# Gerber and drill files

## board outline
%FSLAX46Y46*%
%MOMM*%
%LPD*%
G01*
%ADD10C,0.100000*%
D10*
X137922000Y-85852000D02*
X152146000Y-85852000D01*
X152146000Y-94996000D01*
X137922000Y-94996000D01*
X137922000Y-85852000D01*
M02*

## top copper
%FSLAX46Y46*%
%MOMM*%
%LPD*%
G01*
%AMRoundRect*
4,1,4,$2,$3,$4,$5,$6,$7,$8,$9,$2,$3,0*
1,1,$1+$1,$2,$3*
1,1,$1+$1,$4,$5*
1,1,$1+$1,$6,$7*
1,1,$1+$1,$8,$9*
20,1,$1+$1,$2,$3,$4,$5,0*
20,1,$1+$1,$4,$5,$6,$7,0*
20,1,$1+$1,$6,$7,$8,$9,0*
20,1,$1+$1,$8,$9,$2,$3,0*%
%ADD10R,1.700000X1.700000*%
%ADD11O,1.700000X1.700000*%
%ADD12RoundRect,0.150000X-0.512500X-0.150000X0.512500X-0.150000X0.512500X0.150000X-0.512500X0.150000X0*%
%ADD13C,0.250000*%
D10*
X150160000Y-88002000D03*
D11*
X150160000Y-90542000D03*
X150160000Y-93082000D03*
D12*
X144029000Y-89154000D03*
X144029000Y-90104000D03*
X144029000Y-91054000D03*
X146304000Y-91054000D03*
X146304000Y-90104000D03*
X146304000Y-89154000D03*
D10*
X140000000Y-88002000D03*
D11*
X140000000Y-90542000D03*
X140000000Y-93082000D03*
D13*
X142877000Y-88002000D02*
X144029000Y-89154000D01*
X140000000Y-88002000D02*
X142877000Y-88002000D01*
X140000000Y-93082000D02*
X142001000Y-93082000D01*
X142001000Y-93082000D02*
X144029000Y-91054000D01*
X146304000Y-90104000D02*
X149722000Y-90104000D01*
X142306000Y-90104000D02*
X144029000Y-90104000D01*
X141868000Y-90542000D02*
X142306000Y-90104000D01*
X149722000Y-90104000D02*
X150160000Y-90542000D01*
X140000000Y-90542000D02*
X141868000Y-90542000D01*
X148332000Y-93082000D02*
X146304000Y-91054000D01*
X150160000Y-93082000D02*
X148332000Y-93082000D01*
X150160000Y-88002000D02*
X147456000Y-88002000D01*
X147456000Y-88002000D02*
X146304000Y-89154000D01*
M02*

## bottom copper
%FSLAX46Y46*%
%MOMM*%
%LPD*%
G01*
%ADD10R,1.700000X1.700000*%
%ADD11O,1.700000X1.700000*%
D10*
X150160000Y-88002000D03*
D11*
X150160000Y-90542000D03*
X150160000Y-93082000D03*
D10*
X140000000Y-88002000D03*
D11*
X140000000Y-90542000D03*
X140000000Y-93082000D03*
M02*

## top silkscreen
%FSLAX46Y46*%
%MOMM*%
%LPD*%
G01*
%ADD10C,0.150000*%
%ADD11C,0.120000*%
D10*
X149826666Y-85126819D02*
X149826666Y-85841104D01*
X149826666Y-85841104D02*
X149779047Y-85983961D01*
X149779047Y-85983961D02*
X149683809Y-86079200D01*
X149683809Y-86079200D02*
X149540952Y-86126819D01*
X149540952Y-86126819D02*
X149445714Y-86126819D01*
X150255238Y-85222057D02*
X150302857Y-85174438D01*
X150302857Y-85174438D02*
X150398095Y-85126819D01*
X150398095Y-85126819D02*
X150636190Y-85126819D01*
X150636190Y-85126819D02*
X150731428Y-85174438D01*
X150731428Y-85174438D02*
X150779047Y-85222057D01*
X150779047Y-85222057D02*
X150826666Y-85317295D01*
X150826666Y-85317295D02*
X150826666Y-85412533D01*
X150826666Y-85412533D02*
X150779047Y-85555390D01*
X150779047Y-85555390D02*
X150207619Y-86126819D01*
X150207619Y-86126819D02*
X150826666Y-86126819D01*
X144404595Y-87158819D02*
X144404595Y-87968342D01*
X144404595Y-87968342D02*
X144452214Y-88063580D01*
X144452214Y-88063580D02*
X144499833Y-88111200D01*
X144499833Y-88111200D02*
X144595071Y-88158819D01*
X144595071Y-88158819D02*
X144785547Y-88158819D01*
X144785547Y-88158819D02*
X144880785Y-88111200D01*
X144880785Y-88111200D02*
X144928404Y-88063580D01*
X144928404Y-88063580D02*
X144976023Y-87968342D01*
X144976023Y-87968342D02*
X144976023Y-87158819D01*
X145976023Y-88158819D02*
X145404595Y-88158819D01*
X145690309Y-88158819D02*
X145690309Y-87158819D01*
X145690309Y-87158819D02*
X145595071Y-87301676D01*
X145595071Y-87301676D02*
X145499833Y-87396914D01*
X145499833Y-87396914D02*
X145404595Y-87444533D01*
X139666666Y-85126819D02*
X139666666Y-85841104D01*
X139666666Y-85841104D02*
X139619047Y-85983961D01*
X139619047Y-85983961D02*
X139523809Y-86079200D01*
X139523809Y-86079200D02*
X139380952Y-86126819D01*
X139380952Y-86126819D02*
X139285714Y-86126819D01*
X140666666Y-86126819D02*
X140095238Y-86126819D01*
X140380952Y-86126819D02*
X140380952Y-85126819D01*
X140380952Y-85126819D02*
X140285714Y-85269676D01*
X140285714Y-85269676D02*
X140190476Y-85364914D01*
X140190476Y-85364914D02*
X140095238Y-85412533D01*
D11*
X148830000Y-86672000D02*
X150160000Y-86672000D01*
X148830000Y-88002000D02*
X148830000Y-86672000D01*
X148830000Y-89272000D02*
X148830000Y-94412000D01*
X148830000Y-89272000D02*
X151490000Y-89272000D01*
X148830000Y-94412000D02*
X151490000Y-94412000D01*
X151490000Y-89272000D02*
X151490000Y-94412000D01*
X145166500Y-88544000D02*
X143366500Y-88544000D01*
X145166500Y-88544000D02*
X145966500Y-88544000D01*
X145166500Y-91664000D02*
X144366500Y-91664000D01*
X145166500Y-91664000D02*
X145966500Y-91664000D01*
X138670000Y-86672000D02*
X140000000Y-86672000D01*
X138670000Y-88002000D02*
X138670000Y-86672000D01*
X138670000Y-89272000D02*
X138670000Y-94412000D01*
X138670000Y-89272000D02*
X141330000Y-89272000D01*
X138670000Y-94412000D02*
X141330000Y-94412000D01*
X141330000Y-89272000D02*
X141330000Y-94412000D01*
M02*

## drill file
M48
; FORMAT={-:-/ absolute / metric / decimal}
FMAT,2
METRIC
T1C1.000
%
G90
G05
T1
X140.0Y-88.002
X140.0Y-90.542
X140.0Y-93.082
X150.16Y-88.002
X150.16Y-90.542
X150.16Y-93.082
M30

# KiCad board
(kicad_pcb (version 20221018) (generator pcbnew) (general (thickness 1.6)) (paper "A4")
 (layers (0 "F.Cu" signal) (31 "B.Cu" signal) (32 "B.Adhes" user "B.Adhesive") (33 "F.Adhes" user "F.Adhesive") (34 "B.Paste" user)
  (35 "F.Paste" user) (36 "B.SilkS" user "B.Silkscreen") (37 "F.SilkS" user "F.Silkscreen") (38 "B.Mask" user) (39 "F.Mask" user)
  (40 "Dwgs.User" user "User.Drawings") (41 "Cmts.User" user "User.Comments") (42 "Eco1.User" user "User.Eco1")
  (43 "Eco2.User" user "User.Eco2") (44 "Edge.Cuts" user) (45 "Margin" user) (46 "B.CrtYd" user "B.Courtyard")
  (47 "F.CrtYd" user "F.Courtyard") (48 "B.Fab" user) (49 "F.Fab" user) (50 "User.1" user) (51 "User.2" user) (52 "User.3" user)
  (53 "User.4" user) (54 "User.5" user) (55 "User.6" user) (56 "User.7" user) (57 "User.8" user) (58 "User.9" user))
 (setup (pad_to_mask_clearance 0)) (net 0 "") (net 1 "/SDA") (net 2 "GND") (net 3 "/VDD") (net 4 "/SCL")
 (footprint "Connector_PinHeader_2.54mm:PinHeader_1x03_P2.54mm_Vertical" (layer "F.Cu") (at 150.16 88.002)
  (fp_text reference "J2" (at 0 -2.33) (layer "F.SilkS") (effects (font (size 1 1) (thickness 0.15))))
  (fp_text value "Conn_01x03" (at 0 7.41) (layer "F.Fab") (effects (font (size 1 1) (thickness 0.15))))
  (fp_line (start -1.33 -1.33) (end 0 -1.33) (stroke (width 0.12) (type solid)) (layer "F.SilkS"))
  (fp_line (start -1.33 0) (end -1.33 -1.33) (stroke (width 0.12) (type solid)) (layer "F.SilkS"))
  (fp_line (start -1.33 1.27) (end -1.33 6.41) (stroke (width 0.12) (type solid)) (layer "F.SilkS"))
  (fp_line (start -1.33 1.27) (end 1.33 1.27) (stroke (width 0.12) (type solid)) (layer "F.SilkS"))
  (fp_line (start -1.33 6.41) (end 1.33 6.41) (stroke (width 0.12) (type solid)) (layer "F.SilkS"))
  (fp_line (start 1.33 1.27) (end 1.33 6.41) (stroke (width 0.12) (type solid)) (layer "F.SilkS"))
  (pad "1" thru_hole rect (at 0 0) (size 1.7 1.7) (drill 1) (layers "*.Cu" "*.Mask") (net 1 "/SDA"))
  (pad "2" thru_hole oval (at 0 2.54) (size 1.7 1.7) (drill 1) (layers "*.Cu" "*.Mask") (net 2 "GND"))
  (pad "3" thru_hole oval (at 0 5.08) (size 1.7 1.7) (drill 1) (layers "*.Cu" "*.Mask") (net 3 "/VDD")))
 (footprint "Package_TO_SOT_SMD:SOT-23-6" (layer "F.Cu") (at 145.1665 90.104)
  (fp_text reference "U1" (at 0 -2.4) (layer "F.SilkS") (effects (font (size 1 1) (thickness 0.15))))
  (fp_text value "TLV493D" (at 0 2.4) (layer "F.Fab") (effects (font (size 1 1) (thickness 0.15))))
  (fp_line (start 0 -1.56) (end -1.8 -1.56) (stroke (width 0.12) (type solid)) (layer "F.SilkS"))
  (fp_line (start 0 -1.56) (end 0.8 -1.56) (stroke (width 0.12) (type solid)) (layer "F.SilkS"))
  (fp_line (start 0 1.56) (end -0.8 1.56) (stroke (width 0.12) (type solid)) (layer "F.SilkS"))
  (fp_line (start 0 1.56) (end 0.8 1.56) (stroke (width 0.12) (type solid)) (layer "F.SilkS"))
  (pad "1" smd roundrect (at -1.1375 -0.95) (size 1.325 0.6) (layers "F.Cu" "F.Paste" "F.Mask") (roundrect_rratio 0.25) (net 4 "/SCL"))
  (pad "2" smd roundrect (at -1.1375 0) (size 1.325 0.6) (layers "F.Cu" "F.Paste" "F.Mask") (roundrect_rratio 0.25) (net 2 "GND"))
  (pad "3" smd roundrect (at -1.1375 0.95) (size 1.325 0.6) (layers "F.Cu" "F.Paste" "F.Mask") (roundrect_rratio 0.25) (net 2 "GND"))
  (pad "4" smd roundrect (at 1.1375 0.95) (size 1.325 0.6) (layers "F.Cu" "F.Paste" "F.Mask") (roundrect_rratio 0.25) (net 3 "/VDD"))
  (pad "5" smd roundrect (at 1.1375 0) (size 1.325 0.6) (layers "F.Cu" "F.Paste" "F.Mask") (roundrect_rratio 0.25) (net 2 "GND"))
  (pad "6" smd roundrect (at 1.1375 -0.95) (size 1.325 0.6) (layers "F.Cu" "F.Paste" "F.Mask") (roundrect_rratio 0.25) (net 1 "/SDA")))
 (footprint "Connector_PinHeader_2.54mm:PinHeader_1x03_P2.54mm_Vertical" (layer "F.Cu") (at 140 88.002)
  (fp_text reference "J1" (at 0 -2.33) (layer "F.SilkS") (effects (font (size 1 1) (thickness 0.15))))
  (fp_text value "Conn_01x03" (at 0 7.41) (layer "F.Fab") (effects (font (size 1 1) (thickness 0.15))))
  (fp_line (start -1.33 -1.33) (end 0 -1.33) (stroke (width 0.12) (type solid)) (layer "F.SilkS"))
  (fp_line (start -1.33 0) (end -1.33 -1.33) (stroke (width 0.12) (type solid)) (layer "F.SilkS"))
  (fp_line (start -1.33 1.27) (end -1.33 6.41) (stroke (width 0.12) (type solid)) (layer "F.SilkS"))
  (fp_line (start -1.33 1.27) (end 1.33 1.27) (stroke (width 0.12) (type solid)) (layer "F.SilkS"))
  (fp_line (start -1.33 6.41) (end 1.33 6.41) (stroke (width 0.12) (type solid)) (layer "F.SilkS"))
  (fp_line (start 1.33 1.27) (end 1.33 6.41) (stroke (width 0.12) (type solid)) (layer "F.SilkS"))
  (pad "1" thru_hole rect (at 0 0) (size 1.7 1.7) (drill 1) (layers "*.Cu" "*.Mask") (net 4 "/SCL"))
  (pad "2" thru_hole oval (at 0 2.54) (size 1.7 1.7) (drill 1) (layers "*.Cu" "*.Mask") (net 2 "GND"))
  (pad "3" thru_hole oval (at 0 5.08) (size 1.7 1.7) (drill 1) (layers "*.Cu" "*.Mask") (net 2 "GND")))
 (gr_rect (start 137.922 85.852) (end 152.146 94.996) (stroke (width 0.1) (type default)) (fill none) (layer "Edge.Cuts"))
 (segment (start 142.877 88.002) (end 144.029 89.154) (width 0.25) (layer "F.Cu") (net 4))
 (segment (start 140 88.002) (end 142.877 88.002) (width 0.25) (layer "F.Cu") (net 4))
 (segment (start 140 93.082) (end 142.001 93.082) (width 0.25) (layer "F.Cu") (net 2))
 (segment (start 142.001 93.082) (end 144.029 91.054) (width 0.25) (layer "F.Cu") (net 2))
 (segment (start 146.304 90.104) (end 149.722 90.104) (width 0.25) (layer "F.Cu") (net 2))
 (segment (start 142.306 90.104) (end 144.029 90.104) (width 0.25) (layer "F.Cu") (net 2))
 (segment (start 141.868 90.542) (end 142.306 90.104) (width 0.25) (layer "F.Cu") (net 2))
 (segment (start 149.722 90.104) (end 150.16 90.542) (width 0.25) (layer "F.Cu") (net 2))
 (segment (start 140 90.542) (end 141.868 90.542) (width 0.25) (layer "F.Cu") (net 2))
 (segment (start 148.332 93.082) (end 146.304 91.054) (width 0.25) (layer "F.Cu") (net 3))
 (segment (start 150.16 93.082) (end 148.332 93.082) (width 0.25) (layer "F.Cu") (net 3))
 (segment (start 150.16 88.002) (end 147.456 88.002) (width 0.25) (layer "F.Cu") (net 1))
 (segment (start 147.456 88.002) (end 146.304 89.154) (width 0.25) (layer "F.Cu") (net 1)))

